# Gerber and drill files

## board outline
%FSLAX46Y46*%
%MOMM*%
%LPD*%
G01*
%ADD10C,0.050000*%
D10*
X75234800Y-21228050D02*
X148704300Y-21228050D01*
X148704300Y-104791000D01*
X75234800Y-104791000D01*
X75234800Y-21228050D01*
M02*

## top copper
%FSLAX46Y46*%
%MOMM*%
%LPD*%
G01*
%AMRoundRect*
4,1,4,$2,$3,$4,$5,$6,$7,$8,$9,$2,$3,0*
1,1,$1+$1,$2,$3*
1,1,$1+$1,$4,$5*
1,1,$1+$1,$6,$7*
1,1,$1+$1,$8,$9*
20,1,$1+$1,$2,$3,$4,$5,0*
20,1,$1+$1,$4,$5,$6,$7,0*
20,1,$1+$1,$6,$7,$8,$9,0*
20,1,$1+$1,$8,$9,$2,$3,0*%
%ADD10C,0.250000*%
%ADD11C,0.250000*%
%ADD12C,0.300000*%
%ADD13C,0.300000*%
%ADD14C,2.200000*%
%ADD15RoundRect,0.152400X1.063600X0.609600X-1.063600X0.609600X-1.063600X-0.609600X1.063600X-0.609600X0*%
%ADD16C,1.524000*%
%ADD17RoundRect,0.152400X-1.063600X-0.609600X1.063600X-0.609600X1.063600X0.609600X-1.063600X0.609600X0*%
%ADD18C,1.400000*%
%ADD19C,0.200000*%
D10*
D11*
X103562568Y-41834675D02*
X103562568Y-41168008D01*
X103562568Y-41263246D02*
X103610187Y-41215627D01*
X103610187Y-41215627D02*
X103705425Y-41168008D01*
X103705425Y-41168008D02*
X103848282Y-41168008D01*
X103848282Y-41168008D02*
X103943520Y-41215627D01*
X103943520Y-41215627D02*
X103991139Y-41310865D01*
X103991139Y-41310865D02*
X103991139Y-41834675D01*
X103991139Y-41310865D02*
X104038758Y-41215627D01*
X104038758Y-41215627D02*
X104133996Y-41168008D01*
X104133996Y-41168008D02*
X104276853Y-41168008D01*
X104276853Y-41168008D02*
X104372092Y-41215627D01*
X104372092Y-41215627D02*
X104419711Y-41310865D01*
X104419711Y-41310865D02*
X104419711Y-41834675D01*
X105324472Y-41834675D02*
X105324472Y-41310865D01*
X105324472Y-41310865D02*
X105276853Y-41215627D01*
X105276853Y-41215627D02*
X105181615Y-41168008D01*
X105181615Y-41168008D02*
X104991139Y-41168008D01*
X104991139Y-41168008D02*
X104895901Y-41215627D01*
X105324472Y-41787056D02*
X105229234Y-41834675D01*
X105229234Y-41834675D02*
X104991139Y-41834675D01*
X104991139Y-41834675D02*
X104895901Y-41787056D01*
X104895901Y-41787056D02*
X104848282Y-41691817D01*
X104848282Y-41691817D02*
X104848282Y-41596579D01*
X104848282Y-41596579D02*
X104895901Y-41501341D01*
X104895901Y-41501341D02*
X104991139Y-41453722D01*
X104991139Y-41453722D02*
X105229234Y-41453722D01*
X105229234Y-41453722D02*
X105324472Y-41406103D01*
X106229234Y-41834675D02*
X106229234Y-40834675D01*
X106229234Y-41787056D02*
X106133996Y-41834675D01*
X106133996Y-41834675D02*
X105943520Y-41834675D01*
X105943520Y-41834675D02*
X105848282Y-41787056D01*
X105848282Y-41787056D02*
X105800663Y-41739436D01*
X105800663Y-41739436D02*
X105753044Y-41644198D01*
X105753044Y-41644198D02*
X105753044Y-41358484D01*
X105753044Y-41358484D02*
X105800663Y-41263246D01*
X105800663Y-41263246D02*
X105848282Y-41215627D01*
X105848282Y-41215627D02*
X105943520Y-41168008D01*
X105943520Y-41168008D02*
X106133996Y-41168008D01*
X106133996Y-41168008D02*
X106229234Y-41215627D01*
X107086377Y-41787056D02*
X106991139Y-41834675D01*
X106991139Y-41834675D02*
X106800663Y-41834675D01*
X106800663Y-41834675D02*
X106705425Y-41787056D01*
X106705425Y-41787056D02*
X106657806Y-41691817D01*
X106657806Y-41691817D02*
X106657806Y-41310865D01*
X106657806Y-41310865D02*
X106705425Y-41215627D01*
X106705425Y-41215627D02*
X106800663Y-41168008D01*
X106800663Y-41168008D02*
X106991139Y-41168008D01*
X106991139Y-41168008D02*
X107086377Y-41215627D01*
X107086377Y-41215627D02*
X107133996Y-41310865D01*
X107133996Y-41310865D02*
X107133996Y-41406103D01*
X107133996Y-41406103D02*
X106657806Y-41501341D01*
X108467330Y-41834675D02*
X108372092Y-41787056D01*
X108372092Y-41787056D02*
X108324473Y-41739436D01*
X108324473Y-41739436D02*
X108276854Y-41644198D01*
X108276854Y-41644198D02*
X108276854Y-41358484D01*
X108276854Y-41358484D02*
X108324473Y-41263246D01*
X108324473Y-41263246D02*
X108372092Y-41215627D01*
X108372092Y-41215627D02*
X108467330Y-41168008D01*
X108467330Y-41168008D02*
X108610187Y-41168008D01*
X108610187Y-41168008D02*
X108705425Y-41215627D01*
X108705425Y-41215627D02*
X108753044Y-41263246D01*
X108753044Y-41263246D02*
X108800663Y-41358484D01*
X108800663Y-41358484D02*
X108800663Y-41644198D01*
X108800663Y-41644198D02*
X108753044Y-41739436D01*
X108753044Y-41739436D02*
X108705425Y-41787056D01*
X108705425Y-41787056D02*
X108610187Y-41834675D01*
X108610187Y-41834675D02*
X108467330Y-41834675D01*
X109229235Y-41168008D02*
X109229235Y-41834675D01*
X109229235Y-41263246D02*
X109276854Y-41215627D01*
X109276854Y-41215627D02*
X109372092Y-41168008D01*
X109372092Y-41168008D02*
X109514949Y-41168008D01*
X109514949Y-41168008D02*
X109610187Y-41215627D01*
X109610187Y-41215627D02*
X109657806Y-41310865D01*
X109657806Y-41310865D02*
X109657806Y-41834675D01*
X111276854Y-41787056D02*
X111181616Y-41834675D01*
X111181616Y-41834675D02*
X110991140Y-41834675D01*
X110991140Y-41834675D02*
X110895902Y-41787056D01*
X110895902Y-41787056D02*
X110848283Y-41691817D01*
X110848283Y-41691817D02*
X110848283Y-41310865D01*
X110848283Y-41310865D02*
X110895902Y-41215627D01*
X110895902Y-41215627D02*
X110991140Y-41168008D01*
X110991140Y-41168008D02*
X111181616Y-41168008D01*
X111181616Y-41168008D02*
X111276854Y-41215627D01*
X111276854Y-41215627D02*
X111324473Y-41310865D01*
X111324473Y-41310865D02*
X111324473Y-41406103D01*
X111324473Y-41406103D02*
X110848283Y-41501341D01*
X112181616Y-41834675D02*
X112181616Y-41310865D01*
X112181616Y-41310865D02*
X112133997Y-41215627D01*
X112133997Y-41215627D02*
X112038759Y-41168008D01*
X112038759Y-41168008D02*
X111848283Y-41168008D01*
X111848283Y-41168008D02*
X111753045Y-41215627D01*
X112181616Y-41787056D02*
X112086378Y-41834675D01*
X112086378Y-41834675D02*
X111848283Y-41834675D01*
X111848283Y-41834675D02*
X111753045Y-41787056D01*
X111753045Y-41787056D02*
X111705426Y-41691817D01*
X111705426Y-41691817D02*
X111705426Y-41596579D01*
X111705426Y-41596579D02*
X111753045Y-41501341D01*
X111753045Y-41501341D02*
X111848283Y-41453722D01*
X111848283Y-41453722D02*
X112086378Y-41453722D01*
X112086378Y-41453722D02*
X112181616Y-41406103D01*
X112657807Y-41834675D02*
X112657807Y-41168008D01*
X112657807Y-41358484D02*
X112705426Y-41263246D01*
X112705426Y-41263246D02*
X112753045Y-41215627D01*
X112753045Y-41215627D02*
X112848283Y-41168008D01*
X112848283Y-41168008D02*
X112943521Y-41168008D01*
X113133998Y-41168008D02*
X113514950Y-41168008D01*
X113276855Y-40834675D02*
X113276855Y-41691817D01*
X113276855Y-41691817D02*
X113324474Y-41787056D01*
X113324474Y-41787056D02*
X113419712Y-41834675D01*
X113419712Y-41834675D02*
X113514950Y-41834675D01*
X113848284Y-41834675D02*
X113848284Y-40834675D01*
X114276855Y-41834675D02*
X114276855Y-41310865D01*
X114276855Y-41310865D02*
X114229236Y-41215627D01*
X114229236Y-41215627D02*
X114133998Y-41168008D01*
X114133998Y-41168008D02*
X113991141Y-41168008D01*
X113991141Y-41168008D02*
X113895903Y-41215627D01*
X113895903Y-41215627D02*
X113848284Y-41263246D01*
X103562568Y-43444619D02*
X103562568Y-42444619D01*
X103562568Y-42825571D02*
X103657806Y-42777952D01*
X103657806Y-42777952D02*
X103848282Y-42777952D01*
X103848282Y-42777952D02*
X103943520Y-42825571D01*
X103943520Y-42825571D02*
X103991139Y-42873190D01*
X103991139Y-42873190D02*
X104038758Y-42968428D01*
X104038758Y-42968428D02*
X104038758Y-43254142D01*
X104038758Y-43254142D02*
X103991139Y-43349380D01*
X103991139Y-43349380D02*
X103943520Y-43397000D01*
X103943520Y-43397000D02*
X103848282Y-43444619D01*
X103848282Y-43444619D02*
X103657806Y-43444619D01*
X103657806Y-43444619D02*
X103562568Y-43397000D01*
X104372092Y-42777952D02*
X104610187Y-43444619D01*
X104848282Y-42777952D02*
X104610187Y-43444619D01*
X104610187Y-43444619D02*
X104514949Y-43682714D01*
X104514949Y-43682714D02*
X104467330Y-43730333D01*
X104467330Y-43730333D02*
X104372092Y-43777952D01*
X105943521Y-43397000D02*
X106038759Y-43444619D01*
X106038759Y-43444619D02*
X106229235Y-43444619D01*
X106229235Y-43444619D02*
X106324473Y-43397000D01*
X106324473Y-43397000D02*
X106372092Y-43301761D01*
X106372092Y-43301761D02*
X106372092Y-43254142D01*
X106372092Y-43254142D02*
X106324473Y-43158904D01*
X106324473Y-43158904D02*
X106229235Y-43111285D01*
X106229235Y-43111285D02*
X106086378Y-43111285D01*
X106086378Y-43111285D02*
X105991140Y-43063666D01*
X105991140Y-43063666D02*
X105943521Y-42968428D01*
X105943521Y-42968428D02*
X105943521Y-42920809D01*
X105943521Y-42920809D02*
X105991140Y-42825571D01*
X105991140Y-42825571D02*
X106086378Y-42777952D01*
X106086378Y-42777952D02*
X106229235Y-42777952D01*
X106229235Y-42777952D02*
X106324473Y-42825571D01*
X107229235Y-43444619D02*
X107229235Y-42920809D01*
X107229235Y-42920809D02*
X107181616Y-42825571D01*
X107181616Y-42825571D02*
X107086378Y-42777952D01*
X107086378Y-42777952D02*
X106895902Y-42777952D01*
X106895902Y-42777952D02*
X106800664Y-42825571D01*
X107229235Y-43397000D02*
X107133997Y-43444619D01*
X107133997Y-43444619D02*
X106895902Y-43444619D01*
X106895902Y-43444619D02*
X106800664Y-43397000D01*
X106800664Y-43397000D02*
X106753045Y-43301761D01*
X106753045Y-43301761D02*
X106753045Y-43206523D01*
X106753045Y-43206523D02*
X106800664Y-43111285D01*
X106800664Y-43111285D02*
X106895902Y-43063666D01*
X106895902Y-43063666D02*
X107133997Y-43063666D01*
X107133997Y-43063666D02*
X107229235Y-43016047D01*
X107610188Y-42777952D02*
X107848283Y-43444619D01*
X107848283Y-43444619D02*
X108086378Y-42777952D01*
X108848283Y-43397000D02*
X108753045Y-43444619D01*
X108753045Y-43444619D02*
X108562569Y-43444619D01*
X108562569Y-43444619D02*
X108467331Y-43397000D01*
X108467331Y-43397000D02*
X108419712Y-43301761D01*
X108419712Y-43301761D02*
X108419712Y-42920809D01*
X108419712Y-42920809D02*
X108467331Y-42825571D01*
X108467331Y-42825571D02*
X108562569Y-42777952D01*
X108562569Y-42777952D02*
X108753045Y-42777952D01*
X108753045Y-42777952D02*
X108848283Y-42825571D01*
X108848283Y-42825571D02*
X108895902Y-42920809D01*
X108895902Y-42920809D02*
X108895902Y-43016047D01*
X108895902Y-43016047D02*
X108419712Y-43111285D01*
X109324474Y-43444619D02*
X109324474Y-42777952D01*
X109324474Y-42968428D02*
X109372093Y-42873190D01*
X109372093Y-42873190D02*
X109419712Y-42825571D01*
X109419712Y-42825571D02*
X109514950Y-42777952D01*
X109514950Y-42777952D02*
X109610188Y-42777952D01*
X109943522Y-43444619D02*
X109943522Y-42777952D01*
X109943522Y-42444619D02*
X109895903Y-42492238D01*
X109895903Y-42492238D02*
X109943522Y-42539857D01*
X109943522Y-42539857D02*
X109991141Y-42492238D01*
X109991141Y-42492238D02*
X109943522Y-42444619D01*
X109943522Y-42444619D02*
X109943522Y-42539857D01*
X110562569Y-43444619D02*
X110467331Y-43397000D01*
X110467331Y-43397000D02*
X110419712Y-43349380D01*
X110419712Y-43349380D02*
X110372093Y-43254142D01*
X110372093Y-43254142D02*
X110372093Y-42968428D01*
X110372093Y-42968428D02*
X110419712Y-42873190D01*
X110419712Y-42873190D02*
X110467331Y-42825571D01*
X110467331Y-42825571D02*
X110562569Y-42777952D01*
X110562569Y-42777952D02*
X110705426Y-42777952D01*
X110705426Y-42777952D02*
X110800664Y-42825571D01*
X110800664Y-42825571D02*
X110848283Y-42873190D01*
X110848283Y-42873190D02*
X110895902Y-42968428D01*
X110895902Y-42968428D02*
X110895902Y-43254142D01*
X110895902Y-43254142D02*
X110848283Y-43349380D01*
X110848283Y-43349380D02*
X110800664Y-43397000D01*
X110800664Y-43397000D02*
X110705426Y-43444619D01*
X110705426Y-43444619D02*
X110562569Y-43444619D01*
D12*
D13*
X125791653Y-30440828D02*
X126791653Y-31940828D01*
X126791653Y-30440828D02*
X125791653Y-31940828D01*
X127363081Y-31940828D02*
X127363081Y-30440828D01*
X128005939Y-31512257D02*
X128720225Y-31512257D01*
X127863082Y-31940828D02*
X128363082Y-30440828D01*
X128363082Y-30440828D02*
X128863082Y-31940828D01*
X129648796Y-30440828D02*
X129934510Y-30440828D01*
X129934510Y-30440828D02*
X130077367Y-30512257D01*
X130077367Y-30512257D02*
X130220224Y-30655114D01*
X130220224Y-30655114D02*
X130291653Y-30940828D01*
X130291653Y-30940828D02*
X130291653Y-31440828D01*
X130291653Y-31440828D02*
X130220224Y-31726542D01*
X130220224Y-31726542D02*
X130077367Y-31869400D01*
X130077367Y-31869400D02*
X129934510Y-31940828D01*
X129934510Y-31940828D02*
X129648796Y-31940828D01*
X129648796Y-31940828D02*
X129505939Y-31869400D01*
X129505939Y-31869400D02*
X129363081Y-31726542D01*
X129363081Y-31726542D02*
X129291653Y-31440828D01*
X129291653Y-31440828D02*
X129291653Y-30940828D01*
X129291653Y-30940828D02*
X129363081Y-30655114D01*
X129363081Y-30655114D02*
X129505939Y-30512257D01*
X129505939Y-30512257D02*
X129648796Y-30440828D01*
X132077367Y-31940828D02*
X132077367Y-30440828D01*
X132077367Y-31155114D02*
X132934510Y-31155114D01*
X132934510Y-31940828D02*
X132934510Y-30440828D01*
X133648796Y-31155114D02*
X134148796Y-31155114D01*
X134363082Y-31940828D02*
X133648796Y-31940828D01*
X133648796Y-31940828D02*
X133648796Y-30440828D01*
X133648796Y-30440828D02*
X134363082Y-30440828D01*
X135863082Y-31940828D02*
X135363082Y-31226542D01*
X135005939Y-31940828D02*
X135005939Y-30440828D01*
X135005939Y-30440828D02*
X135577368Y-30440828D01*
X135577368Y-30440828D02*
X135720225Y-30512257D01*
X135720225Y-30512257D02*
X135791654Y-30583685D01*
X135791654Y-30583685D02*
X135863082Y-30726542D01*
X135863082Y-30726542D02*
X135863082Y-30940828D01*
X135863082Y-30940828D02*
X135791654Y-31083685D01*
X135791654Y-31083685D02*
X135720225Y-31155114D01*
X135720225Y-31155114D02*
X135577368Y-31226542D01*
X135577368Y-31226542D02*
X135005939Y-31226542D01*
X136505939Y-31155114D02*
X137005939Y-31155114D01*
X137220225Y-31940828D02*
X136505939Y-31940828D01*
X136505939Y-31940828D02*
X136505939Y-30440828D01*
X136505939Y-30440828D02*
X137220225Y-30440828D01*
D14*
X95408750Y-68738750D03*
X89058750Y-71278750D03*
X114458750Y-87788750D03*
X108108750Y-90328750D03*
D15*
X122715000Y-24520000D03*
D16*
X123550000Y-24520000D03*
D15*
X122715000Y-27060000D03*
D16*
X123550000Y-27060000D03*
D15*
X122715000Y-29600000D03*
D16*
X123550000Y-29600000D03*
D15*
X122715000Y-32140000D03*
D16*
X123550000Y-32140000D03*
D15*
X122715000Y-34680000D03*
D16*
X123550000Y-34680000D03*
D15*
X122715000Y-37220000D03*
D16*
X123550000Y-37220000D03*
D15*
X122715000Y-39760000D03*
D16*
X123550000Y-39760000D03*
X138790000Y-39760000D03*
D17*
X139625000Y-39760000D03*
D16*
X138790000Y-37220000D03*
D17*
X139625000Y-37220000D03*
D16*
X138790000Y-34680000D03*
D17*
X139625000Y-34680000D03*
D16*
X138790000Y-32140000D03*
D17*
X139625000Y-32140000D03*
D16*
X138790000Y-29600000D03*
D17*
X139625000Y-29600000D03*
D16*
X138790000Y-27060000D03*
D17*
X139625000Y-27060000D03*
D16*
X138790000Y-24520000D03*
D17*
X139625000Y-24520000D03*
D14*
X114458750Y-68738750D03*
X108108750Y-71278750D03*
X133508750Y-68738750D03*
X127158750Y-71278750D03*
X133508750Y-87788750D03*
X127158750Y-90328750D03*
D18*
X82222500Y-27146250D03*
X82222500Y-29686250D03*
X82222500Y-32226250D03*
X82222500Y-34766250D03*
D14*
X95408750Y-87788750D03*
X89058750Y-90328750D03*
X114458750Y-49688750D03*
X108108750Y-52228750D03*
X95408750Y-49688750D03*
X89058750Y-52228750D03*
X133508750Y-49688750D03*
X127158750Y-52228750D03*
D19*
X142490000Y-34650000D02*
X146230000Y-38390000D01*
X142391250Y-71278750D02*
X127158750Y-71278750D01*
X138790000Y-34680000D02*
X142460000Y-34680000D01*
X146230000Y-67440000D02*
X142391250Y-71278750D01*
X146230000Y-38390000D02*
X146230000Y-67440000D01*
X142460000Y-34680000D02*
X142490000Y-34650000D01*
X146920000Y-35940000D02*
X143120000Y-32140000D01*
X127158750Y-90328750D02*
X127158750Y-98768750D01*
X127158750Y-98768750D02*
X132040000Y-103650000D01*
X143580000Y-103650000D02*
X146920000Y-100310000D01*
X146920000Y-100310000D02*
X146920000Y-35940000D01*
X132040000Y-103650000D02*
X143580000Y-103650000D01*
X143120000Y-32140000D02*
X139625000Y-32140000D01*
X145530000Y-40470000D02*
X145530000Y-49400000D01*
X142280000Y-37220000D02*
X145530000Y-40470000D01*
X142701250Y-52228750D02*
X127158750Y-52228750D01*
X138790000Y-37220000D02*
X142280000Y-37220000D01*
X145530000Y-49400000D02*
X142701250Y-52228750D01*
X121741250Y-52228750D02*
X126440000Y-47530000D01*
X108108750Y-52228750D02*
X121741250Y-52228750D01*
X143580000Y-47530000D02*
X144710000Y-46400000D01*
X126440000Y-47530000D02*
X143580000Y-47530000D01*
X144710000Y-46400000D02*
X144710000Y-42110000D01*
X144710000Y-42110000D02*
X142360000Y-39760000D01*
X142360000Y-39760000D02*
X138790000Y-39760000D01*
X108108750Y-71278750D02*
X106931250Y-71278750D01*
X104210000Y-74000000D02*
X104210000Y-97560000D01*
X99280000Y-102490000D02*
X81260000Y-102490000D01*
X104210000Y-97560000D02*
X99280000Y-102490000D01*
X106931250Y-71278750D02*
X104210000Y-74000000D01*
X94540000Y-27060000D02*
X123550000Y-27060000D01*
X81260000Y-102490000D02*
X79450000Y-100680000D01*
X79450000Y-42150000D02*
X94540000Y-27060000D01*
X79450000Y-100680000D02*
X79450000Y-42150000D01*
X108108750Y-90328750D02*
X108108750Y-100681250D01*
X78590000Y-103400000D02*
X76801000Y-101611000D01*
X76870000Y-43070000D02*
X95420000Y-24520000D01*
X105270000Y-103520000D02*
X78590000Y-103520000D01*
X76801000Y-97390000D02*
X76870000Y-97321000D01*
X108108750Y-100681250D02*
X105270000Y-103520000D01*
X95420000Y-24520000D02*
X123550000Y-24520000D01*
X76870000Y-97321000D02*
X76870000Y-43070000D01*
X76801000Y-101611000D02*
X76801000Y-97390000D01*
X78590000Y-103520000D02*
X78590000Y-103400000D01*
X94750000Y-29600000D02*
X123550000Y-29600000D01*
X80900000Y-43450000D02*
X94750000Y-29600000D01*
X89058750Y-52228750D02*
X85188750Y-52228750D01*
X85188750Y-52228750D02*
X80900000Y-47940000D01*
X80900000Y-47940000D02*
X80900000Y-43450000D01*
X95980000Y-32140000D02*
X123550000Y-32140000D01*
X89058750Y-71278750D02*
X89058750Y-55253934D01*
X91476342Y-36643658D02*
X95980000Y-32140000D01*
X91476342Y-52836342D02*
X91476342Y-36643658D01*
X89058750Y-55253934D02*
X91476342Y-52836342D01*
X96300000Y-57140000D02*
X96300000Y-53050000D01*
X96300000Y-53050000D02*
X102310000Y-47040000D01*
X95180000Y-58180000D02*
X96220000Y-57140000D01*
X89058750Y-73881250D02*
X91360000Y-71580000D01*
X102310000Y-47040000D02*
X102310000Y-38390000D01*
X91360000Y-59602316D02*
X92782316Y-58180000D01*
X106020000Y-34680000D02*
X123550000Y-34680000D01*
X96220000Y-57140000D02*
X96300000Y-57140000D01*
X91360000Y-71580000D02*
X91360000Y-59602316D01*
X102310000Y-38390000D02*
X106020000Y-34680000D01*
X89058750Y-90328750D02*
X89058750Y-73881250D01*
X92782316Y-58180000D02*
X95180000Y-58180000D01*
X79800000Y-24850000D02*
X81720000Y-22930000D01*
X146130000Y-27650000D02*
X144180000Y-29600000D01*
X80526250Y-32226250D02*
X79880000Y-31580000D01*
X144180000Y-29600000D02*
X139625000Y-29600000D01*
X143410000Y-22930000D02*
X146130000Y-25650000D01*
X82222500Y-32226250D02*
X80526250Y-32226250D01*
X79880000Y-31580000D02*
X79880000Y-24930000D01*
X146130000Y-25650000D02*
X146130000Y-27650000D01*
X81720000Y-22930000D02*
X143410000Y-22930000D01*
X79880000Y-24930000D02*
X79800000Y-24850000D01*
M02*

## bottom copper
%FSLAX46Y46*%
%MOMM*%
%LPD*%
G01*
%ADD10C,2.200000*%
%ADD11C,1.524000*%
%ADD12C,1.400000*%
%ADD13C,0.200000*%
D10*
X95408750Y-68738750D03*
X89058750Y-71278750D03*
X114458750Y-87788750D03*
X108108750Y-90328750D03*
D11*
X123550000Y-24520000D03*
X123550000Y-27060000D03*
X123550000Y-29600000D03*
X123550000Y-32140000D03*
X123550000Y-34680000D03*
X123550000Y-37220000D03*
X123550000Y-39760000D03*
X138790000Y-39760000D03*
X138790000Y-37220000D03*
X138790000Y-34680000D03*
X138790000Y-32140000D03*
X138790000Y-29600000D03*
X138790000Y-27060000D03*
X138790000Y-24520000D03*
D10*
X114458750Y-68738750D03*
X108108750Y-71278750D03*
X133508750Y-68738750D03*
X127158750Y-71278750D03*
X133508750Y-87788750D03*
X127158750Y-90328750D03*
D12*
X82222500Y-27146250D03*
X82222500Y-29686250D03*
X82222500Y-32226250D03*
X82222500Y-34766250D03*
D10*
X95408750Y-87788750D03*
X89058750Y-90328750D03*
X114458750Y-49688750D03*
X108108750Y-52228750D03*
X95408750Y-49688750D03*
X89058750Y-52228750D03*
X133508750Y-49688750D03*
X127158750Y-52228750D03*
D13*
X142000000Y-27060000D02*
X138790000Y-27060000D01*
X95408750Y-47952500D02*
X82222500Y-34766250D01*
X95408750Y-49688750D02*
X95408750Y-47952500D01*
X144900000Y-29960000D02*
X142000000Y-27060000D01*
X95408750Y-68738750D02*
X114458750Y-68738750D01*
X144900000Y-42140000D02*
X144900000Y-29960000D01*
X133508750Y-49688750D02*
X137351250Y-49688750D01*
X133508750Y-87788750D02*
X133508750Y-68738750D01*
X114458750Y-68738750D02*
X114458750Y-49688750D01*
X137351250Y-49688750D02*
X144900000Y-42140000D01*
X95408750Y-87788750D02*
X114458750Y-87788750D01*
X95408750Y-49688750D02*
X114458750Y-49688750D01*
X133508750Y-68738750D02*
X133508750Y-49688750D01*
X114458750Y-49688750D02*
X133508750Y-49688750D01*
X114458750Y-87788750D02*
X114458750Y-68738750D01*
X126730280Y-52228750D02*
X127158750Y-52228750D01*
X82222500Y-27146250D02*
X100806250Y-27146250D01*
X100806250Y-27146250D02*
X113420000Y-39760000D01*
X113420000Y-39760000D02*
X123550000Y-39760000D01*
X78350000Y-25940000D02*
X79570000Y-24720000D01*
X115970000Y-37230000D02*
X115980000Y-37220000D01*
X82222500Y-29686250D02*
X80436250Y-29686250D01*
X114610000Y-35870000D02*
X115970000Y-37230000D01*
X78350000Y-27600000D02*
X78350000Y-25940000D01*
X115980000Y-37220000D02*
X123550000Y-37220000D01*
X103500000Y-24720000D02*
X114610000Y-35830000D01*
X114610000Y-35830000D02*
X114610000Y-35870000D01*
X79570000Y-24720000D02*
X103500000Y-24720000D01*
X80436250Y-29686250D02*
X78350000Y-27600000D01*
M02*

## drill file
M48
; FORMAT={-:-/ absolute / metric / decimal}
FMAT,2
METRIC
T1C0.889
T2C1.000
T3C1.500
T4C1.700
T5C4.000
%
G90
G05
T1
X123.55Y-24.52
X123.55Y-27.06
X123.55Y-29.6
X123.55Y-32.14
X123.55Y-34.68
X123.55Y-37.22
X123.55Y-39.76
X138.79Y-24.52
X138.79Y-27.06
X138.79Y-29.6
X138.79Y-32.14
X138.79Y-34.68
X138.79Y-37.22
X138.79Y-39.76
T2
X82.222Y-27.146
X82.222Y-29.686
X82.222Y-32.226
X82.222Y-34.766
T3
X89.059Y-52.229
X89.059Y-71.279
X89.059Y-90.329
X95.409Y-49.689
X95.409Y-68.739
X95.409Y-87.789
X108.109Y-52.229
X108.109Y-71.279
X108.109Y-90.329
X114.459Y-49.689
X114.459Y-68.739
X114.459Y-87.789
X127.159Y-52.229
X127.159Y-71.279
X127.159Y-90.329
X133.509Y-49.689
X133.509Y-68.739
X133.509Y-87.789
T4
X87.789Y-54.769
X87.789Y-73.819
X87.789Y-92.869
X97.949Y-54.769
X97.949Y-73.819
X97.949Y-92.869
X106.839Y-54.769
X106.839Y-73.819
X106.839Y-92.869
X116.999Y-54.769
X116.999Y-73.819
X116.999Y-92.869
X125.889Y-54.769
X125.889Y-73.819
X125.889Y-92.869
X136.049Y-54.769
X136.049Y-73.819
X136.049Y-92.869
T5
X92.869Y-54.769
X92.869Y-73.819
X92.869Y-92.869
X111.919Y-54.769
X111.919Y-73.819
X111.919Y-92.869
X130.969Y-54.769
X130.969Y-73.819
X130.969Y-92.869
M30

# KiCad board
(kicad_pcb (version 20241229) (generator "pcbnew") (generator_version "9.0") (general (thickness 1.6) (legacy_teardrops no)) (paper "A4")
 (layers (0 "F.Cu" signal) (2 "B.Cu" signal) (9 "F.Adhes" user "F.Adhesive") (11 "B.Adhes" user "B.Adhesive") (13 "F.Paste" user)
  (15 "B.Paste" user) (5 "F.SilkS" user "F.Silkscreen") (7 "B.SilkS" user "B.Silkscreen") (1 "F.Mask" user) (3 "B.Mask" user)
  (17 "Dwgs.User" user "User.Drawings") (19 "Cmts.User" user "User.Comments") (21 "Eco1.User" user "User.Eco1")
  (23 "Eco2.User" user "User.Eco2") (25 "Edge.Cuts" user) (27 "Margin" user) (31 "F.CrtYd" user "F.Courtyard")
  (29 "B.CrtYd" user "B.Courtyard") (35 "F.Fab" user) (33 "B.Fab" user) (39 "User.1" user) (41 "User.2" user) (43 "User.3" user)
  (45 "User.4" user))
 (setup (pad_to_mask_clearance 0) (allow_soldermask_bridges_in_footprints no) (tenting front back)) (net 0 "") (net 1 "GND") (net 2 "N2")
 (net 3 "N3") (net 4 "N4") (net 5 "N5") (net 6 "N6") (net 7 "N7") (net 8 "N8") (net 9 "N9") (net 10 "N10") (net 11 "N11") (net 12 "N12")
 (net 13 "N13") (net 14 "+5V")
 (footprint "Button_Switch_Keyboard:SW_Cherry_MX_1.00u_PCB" (layer "F.Cu") (at 95.40875 68.73875)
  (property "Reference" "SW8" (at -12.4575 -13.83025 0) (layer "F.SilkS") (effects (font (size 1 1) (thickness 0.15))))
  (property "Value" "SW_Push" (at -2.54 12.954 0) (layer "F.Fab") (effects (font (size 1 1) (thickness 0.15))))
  (pad "" np_thru_hole circle (at -7.62 5.08) (size 1.7 1.7) (drill 1.7) (layers "*.Cu" "*.Mask"))
  (pad "" np_thru_hole circle (at -2.54 5.08) (size 4 4) (drill 4) (layers "*.Cu" "*.Mask"))
  (pad "" np_thru_hole circle (at 2.54 5.08) (size 1.7 1.7) (drill 1.7) (layers "*.Cu" "*.Mask"))
  (pad "1" thru_hole circle (at 0 0) (size 2.2 2.2) (drill 1.5) (layers "*.Cu" "*.Mask") (remove_unused_layers no) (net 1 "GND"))
  (pad "2" thru_hole circle (at -6.35 2.54) (size 2.2 2.2) (drill 1.5) (layers "*.Cu" "*.Mask") (remove_unused_layers no) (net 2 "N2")))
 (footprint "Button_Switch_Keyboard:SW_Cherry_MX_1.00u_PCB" (layer "F.Cu") (at 114.45875 87.78875)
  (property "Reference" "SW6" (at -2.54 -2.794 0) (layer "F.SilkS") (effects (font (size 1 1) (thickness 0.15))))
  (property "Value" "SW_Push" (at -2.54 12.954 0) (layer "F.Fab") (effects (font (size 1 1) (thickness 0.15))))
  (pad "" np_thru_hole circle (at -7.62 5.08) (size 1.7 1.7) (drill 1.7) (layers "*.Cu" "*.Mask"))
  (pad "" np_thru_hole circle (at -2.54 5.08) (size 4 4) (drill 4) (layers "*.Cu" "*.Mask"))
  (pad "" np_thru_hole circle (at 2.54 5.08) (size 1.7 1.7) (drill 1.7) (layers "*.Cu" "*.Mask"))
  (pad "1" thru_hole circle (at 0 0) (size 2.2 2.2) (drill 1.5) (layers "*.Cu" "*.Mask") (remove_unused_layers no) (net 1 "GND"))
  (pad "2" thru_hole circle (at -6.35 2.54) (size 2.2 2.2) (drill 1.5) (layers "*.Cu" "*.Mask") (remove_unused_layers no) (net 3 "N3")))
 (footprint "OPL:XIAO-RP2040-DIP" (layer "F.Cu") (at 131.17 32.14)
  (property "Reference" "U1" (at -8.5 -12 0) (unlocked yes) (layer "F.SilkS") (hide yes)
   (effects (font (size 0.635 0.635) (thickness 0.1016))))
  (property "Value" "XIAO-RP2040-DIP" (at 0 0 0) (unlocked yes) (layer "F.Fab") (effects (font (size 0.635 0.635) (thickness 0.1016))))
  (pad "1" smd roundrect (at -8.455 -7.62 180) (size 2.432 1.524) (layers "F.Cu" "F.Mask") (roundrect_rratio 0.1) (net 3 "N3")
   (thermal_bridge_angle 45))
  (pad "1" thru_hole circle (at -7.62 -7.62 180) (size 1.524 1.524) (drill 0.889) (layers "*.Cu" "*.Mask") (remove_unused_layers no)
   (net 3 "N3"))
  (pad "2" smd roundrect (at -8.455 -5.08 180) (size 2.432 1.524) (layers "F.Cu" "F.Mask") (roundrect_rratio 0.1) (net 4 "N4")
   (thermal_bridge_angle 45))
  (pad "2" thru_hole circle (at -7.62 -5.08 180) (size 1.524 1.524) (drill 0.889) (layers "*.Cu" "*.Mask") (remove_unused_layers no)
   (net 4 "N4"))
  (pad "3" smd roundrect (at -8.455 -2.54 180) (size 2.432 1.524) (layers "F.Cu" "F.Mask") (roundrect_rratio 0.1) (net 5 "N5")
   (thermal_bridge_angle 45))
  (pad "3" thru_hole circle (at -7.62 -2.54 180) (size 1.524 1.524) (drill 0.889) (layers "*.Cu" "*.Mask") (remove_unused_layers no)
   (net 5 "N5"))
  (pad "4" smd roundrect (at -8.455 0 180) (size 2.432 1.524) (layers "F.Cu" "F.Mask") (roundrect_rratio 0.1) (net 2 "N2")
   (thermal_bridge_angle 45))
  (pad "4" thru_hole circle (at -7.62 0 180) (size 1.524 1.524) (drill 0.889) (layers "*.Cu" "*.Mask") (remove_unused_layers no)
   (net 2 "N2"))
  (pad "5" smd roundrect (at -8.455 2.54 180) (size 2.432 1.524) (layers "F.Cu" "F.Mask") (roundrect_rratio 0.1) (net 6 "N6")
   (thermal_bridge_angle 45))
  (pad "5" thru_hole circle (at -7.62 2.54 180) (size 1.524 1.524) (drill 0.889) (layers "*.Cu" "*.Mask") (remove_unused_layers no)
   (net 6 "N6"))
  (pad "6" smd roundrect (at -8.455 5.08 180) (size 2.432 1.524) (layers "F.Cu" "F.Mask") (roundrect_rratio 0.1) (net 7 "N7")
   (thermal_bridge_angle 45))
  (pad "6" thru_hole circle (at -7.62 5.08 180) (size 1.524 1.524) (drill 0.889) (layers "*.Cu" "*.Mask") (remove_unused_layers no)
   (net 7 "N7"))
  (pad "7" smd roundrect (at -8.455 7.62 180) (size 2.432 1.524) (layers "F.Cu" "F.Mask") (roundrect_rratio 0.1) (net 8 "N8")
   (thermal_bridge_angle 45))
  (pad "7" thru_hole circle (at -7.62 7.62 180) (size 1.524 1.524) (drill 0.889) (layers "*.Cu" "*.Mask") (remove_unused_layers no)
   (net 8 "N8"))
  (pad "8" thru_hole circle (at 7.62 7.62) (size 1.524 1.524) (drill 0.889) (layers "*.Cu" "*.Mask") (remove_unused_layers no) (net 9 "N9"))
  (pad "8" smd roundrect (at 8.455 7.62) (size 2.432 1.524) (layers "F.Cu" "F.Mask") (roundrect_rratio 0.1) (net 9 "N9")
   (thermal_bridge_angle 45))
  (pad "9" thru_hole circle (at 7.62 5.08) (size 1.524 1.524) (drill 0.889) (layers "*.Cu" "*.Mask") (remove_unused_layers no)
   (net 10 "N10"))
  (pad "9" smd roundrect (at 8.455 5.08) (size 2.432 1.524) (layers "F.Cu" "F.Mask") (roundrect_rratio 0.1) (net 10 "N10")
   (thermal_bridge_angle 45))
  (pad "10" thru_hole circle (at 7.62 2.54) (size 1.524 1.524) (drill 0.889) (layers "*.Cu" "*.Mask") (remove_unused_layers no)
   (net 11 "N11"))
  (pad "10" smd roundrect (at 8.455 2.54) (size 2.432 1.524) (layers "F.Cu" "F.Mask") (roundrect_rratio 0.1) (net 11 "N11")
   (thermal_bridge_angle 45))
  (pad "11" thru_hole circle (at 7.62 0) (size 1.524 1.524) (drill 0.889) (layers "*.Cu" "*.Mask") (remove_unused_layers no) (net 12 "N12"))
  (pad "11" smd roundrect (at 8.455 0) (size 2.432 1.524) (layers "F.Cu" "F.Mask") (roundrect_rratio 0.1) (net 12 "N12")
   (thermal_bridge_angle 45))
  (pad "12" thru_hole circle (at 7.62 -2.54) (size 1.524 1.524) (drill 0.889) (layers "*.Cu" "*.Mask") (remove_unused_layers no)
   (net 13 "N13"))
  (pad "12" smd roundrect (at 8.455 -2.54) (size 2.432 1.524) (layers "F.Cu" "F.Mask") (roundrect_rratio 0.1) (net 13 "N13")
   (thermal_bridge_angle 45))
  (pad "13" thru_hole circle (at 7.62 -5.08) (size 1.524 1.524) (drill 0.889) (layers "*.Cu" "*.Mask") (remove_unused_layers no)
   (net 1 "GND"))
  (pad "13" smd roundrect (at 8.455 -5.08) (size 2.432 1.524) (layers "F.Cu" "F.Mask") (roundrect_rratio 0.1) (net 1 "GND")
   (thermal_bridge_angle 45))
  (pad "14" thru_hole circle (at 7.62 -7.62) (size 1.524 1.524) (drill 0.889) (layers "*.Cu" "*.Mask") (remove_unused_layers no)
   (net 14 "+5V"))
  (pad "14" smd roundrect (at 8.455 -7.62) (size 2.432 1.524) (layers "F.Cu" "F.Mask") (roundrect_rratio 0.1) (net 14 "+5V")
   (thermal_bridge_angle 45)))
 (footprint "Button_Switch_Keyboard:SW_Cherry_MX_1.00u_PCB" (layer "F.Cu") (at 114.45875 68.73875)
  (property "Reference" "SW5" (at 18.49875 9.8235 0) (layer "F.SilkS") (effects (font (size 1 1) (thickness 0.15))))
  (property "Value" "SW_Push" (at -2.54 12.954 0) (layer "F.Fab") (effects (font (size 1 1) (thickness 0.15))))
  (pad "" np_thru_hole circle (at -7.62 5.08) (size 1.7 1.7) (drill 1.7) (layers "*.Cu" "*.Mask"))
  (pad "" np_thru_hole circle (at -2.54 5.08) (size 4 4) (drill 4) (layers "*.Cu" "*.Mask"))
  (pad "" np_thru_hole circle (at 2.54 5.08) (size 1.7 1.7) (drill 1.7) (layers "*.Cu" "*.Mask"))
  (pad "1" thru_hole circle (at 0 0) (size 2.2 2.2) (drill 1.5) (layers "*.Cu" "*.Mask") (remove_unused_layers no) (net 1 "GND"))
  (pad "2" thru_hole circle (at -6.35 2.54) (size 2.2 2.2) (drill 1.5) (layers "*.Cu" "*.Mask") (remove_unused_layers no) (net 4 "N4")))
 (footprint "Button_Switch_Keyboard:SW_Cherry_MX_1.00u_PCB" (layer "F.Cu") (at 133.50875 68.73875)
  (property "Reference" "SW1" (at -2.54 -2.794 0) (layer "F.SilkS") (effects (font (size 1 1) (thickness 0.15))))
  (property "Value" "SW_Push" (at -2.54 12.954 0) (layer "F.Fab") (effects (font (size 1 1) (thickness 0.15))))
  (pad "" np_thru_hole circle (at -7.62 5.08) (size 1.7 1.7) (drill 1.7) (layers "*.Cu" "*.Mask"))
  (pad "" np_thru_hole circle (at -2.54 5.08) (size 4 4) (drill 4) (layers "*.Cu" "*.Mask"))
  (pad "" np_thru_hole circle (at 2.54 5.08) (size 1.7 1.7) (drill 1.7) (layers "*.Cu" "*.Mask"))
  (pad "1" thru_hole circle (at 0 0) (size 2.2 2.2) (drill 1.5) (layers "*.Cu" "*.Mask") (remove_unused_layers no) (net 1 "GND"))
  (pad "2" thru_hole circle (at -6.35 2.54) (size 2.2 2.2) (drill 1.5) (layers "*.Cu" "*.Mask") (remove_unused_layers no) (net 11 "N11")))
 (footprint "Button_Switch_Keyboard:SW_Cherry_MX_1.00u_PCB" (layer "F.Cu") (at 133.50875 87.78875)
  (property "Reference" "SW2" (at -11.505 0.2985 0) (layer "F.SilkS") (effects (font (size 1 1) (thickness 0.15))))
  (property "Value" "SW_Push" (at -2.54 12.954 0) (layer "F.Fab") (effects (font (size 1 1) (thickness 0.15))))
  (pad "" np_thru_hole circle (at -7.62 5.08) (size 1.7 1.7) (drill 1.7) (layers "*.Cu" "*.Mask"))
  (pad "" np_thru_hole circle (at -2.54 5.08) (size 4 4) (drill 4) (layers "*.Cu" "*.Mask"))
  (pad "" np_thru_hole circle (at 2.54 5.08) (size 1.7 1.7) (drill 1.7) (layers "*.Cu" "*.Mask"))
  (pad "1" thru_hole circle (at 0 0) (size 2.2 2.2) (drill 1.5) (layers "*.Cu" "*.Mask") (remove_unused_layers no) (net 1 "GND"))
  (pad "2" thru_hole circle (at -6.35 2.54) (size 2.2 2.2) (drill 1.5) (layers "*.Cu" "*.Mask") (remove_unused_layers no) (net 12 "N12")))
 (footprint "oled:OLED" (layer "F.Cu") (at 82.2225 30.95625 -90)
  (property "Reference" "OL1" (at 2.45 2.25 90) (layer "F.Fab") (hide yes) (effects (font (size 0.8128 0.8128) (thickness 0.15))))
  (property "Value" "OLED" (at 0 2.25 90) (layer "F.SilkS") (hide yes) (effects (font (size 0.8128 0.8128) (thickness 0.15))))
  (pad "1" thru_hole circle (at -3.81 0 270) (size 1.4 1.4) (drill 1) (layers "*.Cu" "*.Mask") (remove_unused_layers no) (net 8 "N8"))
  (pad "2" thru_hole circle (at -1.27 0 270) (size 1.4 1.4) (drill 1) (layers "*.Cu" "*.Mask") (remove_unused_layers no) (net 7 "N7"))
  (pad "3" thru_hole circle (at 1.27 0 270) (size 1.4 1.4) (drill 1) (layers "*.Cu" "*.Mask") (remove_unused_layers no) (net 13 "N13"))
  (pad "4" thru_hole circle (at 3.81 0 270) (size 1.4 1.4) (drill 1) (layers "*.Cu" "*.Mask") (remove_unused_layers no) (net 1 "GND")))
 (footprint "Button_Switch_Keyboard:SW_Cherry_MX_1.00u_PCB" (layer "F.Cu") (at 95.40875 87.78875)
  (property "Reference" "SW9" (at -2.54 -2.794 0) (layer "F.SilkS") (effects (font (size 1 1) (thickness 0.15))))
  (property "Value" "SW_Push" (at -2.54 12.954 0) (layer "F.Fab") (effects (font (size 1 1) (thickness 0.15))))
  (pad "" np_thru_hole circle (at -7.62 5.08) (size 1.7 1.7) (drill 1.7) (layers "*.Cu" "*.Mask"))
  (pad "" np_thru_hole circle (at -2.54 5.08) (size 4 4) (drill 4) (layers "*.Cu" "*.Mask"))
  (pad "" np_thru_hole circle (at 2.54 5.08) (size 1.7 1.7) (drill 1.7) (layers "*.Cu" "*.Mask"))
  (pad "1" thru_hole circle (at 0 0) (size 2.2 2.2) (drill 1.5) (layers "*.Cu" "*.Mask") (remove_unused_layers no) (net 1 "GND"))
  (pad "2" thru_hole circle (at -6.35 2.54) (size 2.2 2.2) (drill 1.5) (layers "*.Cu" "*.Mask") (remove_unused_layers no) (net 6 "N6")))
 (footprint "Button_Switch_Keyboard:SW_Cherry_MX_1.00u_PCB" (layer "F.Cu") (at 114.45875 49.68875)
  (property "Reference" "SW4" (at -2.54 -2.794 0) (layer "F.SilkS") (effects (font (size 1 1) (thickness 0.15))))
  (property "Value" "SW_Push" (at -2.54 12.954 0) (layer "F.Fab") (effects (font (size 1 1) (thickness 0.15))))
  (pad "" np_thru_hole circle (at -7.62 5.08) (size 1.7 1.7) (drill 1.7) (layers "*.Cu" "*.Mask"))
  (pad "" np_thru_hole circle (at -2.54 5.08) (size 4 4) (drill 4) (layers "*.Cu" "*.Mask"))
  (pad "" np_thru_hole circle (at 2.54 5.08) (size 1.7 1.7) (drill 1.7) (layers "*.Cu" "*.Mask"))
  (pad "1" thru_hole circle (at 0 0) (size 2.2 2.2) (drill 1.5) (layers "*.Cu" "*.Mask") (remove_unused_layers no) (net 1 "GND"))
  (pad "2" thru_hole circle (at -6.35 2.54) (size 2.2 2.2) (drill 1.5) (layers "*.Cu" "*.Mask") (remove_unused_layers no) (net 9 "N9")))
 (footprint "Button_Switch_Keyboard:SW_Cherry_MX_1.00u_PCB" (layer "F.Cu") (at 95.40875 49.68875)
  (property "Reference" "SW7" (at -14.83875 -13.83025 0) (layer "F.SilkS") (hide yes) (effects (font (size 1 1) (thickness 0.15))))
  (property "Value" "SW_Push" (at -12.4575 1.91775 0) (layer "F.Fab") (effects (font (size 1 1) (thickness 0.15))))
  (pad "" np_thru_hole circle (at -7.62 5.08) (size 1.7 1.7) (drill 1.7) (layers "*.Cu" "*.Mask"))
  (pad "" np_thru_hole circle (at -2.54 5.08) (size 4 4) (drill 4) (layers "*.Cu" "*.Mask"))
  (pad "" np_thru_hole circle (at 2.54 5.08) (size 1.7 1.7) (drill 1.7) (layers "*.Cu" "*.Mask"))
  (pad "1" thru_hole circle (at 0 0) (size 2.2 2.2) (drill 1.5) (layers "*.Cu" "*.Mask") (remove_unused_layers no) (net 1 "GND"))
  (pad "2" thru_hole circle (at -6.35 2.54) (size 2.2 2.2) (drill 1.5) (layers "*.Cu" "*.Mask") (remove_unused_layers no) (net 5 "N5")))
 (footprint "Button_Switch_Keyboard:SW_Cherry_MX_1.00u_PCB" (layer "F.Cu") (at 133.50875 49.68875)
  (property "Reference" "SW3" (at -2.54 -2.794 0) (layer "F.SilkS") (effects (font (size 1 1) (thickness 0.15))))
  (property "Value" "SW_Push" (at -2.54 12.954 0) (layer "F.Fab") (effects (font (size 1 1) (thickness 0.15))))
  (pad "" np_thru_hole circle (at -7.62 5.08) (size 1.7 1.7) (drill 1.7) (layers "*.Cu" "*.Mask"))
  (pad "" np_thru_hole circle (at -2.54 5.08) (size 4 4) (drill 4) (layers "*.Cu" "*.Mask"))
  (pad "" np_thru_hole circle (at 2.54 5.08) (size 1.7 1.7) (drill 1.7) (layers "*.Cu" "*.Mask"))
  (pad "1" thru_hole circle (at 0 0) (size 2.2 2.2) (drill 1.5) (layers "*.Cu" "*.Mask") (remove_unused_layers no) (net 1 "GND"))
  (pad "2" thru_hole circle (at -6.35 2.54) (size 2.2 2.2) (drill 1.5) (layers "*.Cu" "*.Mask") (remove_unused_layers no) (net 10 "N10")))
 (gr_rect (start 75.2348 21.22805) (end 148.7043 104.791) (stroke (width 0.05) (type default)) (fill no) (layer "Edge.Cuts"))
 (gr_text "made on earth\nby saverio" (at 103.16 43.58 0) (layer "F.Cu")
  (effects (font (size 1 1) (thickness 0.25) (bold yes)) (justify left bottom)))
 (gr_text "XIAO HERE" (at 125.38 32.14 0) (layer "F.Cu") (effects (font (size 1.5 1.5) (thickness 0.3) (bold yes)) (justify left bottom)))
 (segment (start 142 27.06) (end 138.79 27.06) (width 0.2) (layer "B.Cu") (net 1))
 (segment (start 95.40875 47.9525) (end 82.2225 34.76625) (width 0.2) (layer "B.Cu") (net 1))
 (segment (start 95.40875 49.68875) (end 95.40875 47.9525) (width 0.2) (layer "B.Cu") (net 1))
 (segment (start 144.9 29.96) (end 142 27.06) (width 0.2) (layer "B.Cu") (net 1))
 (segment (start 95.40875 68.73875) (end 114.45875 68.73875) (width 0.2) (layer "B.Cu") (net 1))
 (segment (start 144.9 42.14) (end 144.9 29.96) (width 0.2) (layer "B.Cu") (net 1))
 (segment (start 133.50875 49.68875) (end 137.35125 49.68875) (width 0.2) (layer "B.Cu") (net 1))
 (segment (start 133.50875 87.78875) (end 133.50875 68.73875) (width 0.2) (layer "B.Cu") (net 1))
 (segment (start 114.45875 68.73875) (end 114.45875 49.68875) (width 0.2) (layer "B.Cu") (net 1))
 (segment (start 137.35125 49.68875) (end 144.9 42.14) (width 0.2) (layer "B.Cu") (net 1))
 (segment (start 95.40875 87.78875) (end 114.45875 87.78875) (width 0.2) (layer "B.Cu") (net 1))
 (segment (start 95.40875 49.68875) (end 114.45875 49.68875) (width 0.2) (layer "B.Cu") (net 1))
 (segment (start 133.50875 68.73875) (end 133.50875 49.68875) (width 0.2) (layer "B.Cu") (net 1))
 (segment (start 114.45875 49.68875) (end 133.50875 49.68875) (width 0.2) (layer "B.Cu") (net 1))
 (segment (start 114.45875 87.78875) (end 114.45875 68.73875) (width 0.2) (layer "B.Cu") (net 1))
 (segment (start 142.49 34.65) (end 146.23 38.39) (width 0.2) (layer "F.Cu") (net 11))
 (segment (start 142.39125 71.27875) (end 127.15875 71.27875) (width 0.2) (layer "F.Cu") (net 11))
 (segment (start 138.79 34.68) (end 142.46 34.68) (width 0.2) (layer "F.Cu") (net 11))
 (segment (start 146.23 67.44) (end 142.39125 71.27875) (width 0.2) (layer "F.Cu") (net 11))
 (segment (start 146.23 38.39) (end 146.23 67.44) (width 0.2) (layer "F.Cu") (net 11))
 (segment (start 142.46 34.68) (end 142.49 34.65) (width 0.2) (layer "F.Cu") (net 11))
 (segment (start 146.92 35.94) (end 143.12 32.14) (width 0.2) (layer "F.Cu") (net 12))
 (segment (start 127.15875 90.32875) (end 127.15875 98.76875) (width 0.2) (layer "F.Cu") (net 12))
 (segment (start 127.15875 98.76875) (end 132.04 103.65) (width 0.2) (layer "F.Cu") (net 12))
 (segment (start 143.58 103.65) (end 146.92 100.31) (width 0.2) (layer "F.Cu") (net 12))
 (segment (start 146.92 100.31) (end 146.92 35.94) (width 0.2) (layer "F.Cu") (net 12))
 (segment (start 132.04 103.65) (end 143.58 103.65) (width 0.2) (layer "F.Cu") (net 12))
 (segment (start 143.12 32.14) (end 139.625 32.14) (width 0.2) (layer "F.Cu") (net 12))
 (segment (start 145.53 40.47) (end 145.53 49.4) (width 0.2) (layer "F.Cu") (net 10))
 (segment (start 142.28 37.22) (end 145.53 40.47) (width 0.2) (layer "F.Cu") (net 10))
 (segment (start 142.70125 52.22875) (end 127.15875 52.22875) (width 0.2) (layer "F.Cu") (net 10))
 (segment (start 138.79 37.22) (end 142.28 37.22) (width 0.2) (layer "F.Cu") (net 10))
 (segment (start 145.53 49.4) (end 142.70125 52.22875) (width 0.2) (layer "F.Cu") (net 10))
 (segment (start 126.73028 52.22875) (end 127.15875 52.22875) (width 0.2) (layer "B.Cu") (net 10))
 (segment (start 121.74125 52.22875) (end 126.44 47.53) (width 0.2) (layer "F.Cu") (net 9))
 (segment (start 108.10875 52.22875) (end 121.74125 52.22875) (width 0.2) (layer "F.Cu") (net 9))
 (segment (start 143.58 47.53) (end 144.71 46.4) (width 0.2) (layer "F.Cu") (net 9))
 (segment (start 126.44 47.53) (end 143.58 47.53) (width 0.2) (layer "F.Cu") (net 9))
 (segment (start 144.71 46.4) (end 144.71 42.11) (width 0.2) (layer "F.Cu") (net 9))
 (segment (start 144.71 42.11) (end 142.36 39.76) (width 0.2) (layer "F.Cu") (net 9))
 (segment (start 142.36 39.76) (end 138.79 39.76) (width 0.2) (layer "F.Cu") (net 9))
 (segment (start 108.10875 71.27875) (end 106.93125 71.27875) (width 0.2) (layer "F.Cu") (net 4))
 (segment (start 104.21 74) (end 104.21 97.56) (width 0.2) (layer "F.Cu") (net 4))
 (segment (start 99.28 102.49) (end 81.26 102.49) (width 0.2) (layer "F.Cu") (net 4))
 (segment (start 104.21 97.56) (end 99.28 102.49) (width 0.2) (layer "F.Cu") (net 4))
 (segment (start 106.93125 71.27875) (end 104.21 74) (width 0.2) (layer "F.Cu") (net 4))
 (segment (start 94.54 27.06) (end 123.55 27.06) (width 0.2) (layer "F.Cu") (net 4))
 (segment (start 81.26 102.49) (end 79.45 100.68) (width 0.2) (layer "F.Cu") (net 4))
 (segment (start 79.45 42.15) (end 94.54 27.06) (width 0.2) (layer "F.Cu") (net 4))
 (segment (start 79.45 100.68) (end 79.45 42.15) (width 0.2) (layer "F.Cu") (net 4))
 (segment (start 108.10875 90.32875) (end 108.10875 100.68125) (width 0.2) (layer "F.Cu") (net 3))
 (segment (start 78.59 103.4) (end 76.801 101.611) (width 0.2) (layer "F.Cu") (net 3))
 (segment (start 76.87 43.07) (end 95.42 24.52) (width 0.2) (layer "F.Cu") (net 3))
 (segment (start 105.27 103.52) (end 78.59 103.52) (width 0.2) (layer "F.Cu") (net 3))
 (segment (start 76.801 97.39) (end 76.87 97.321) (width 0.2) (layer "F.Cu") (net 3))
 (segment (start 108.10875 100.68125) (end 105.27 103.52) (width 0.2) (layer "F.Cu") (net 3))
 (segment (start 95.42 24.52) (end 123.55 24.52) (width 0.2) (layer "F.Cu") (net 3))
 (segment (start 76.87 97.321) (end 76.87 43.07) (width 0.2) (layer "F.Cu") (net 3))
 (segment (start 76.801 101.611) (end 76.801 97.39) (width 0.2) (layer "F.Cu") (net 3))
 (segment (start 78.59 103.52) (end 78.59 103.4) (width 0.2) (layer "F.Cu") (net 3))
 (segment (start 94.75 29.6) (end 123.55 29.6) (width 0.2) (layer "F.Cu") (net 5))
 (segment (start 80.9 43.45) (end 94.75 29.6) (width 0.2) (layer "F.Cu") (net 5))
 (segment (start 89.05875 52.22875) (end 85.18875 52.22875) (width 0.2) (layer "F.Cu") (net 5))
 (segment (start 85.18875 52.22875) (end 80.9 47.94) (width 0.2) (layer "F.Cu") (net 5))
 (segment (start 80.9 47.94) (end 80.9 43.45) (width 0.2) (layer "F.Cu") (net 5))
 (segment (start 95.98 32.14) (end 123.55 32.14) (width 0.2) (layer "F.Cu") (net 2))
 (segment (start 89.05875 71.27875) (end 89.05875 55.253934) (width 0.2) (layer "F.Cu") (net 2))
 (segment (start 91.476342 36.643658) (end 95.98 32.14) (width 0.2) (layer "F.Cu") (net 2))
 (segment (start 91.476342 52.836342) (end 91.476342 36.643658) (width 0.2) (layer "F.Cu") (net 2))
 (segment (start 89.05875 55.253934) (end 91.476342 52.836342) (width 0.2) (layer "F.Cu") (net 2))
 (segment (start 96.3 57.14) (end 96.3 53.05) (width 0.2) (layer "F.Cu") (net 6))
 (segment (start 96.3 53.05) (end 102.31 47.04) (width 0.2) (layer "F.Cu") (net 6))
 (segment (start 95.18 58.18) (end 96.22 57.14) (width 0.2) (layer "F.Cu") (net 6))
 (segment (start 89.05875 73.88125) (end 91.36 71.58) (width 0.2) (layer "F.Cu") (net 6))
 (segment (start 102.31 47.04) (end 102.31 38.39) (width 0.2) (layer "F.Cu") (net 6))
 (segment (start 91.36 59.602316) (end 92.782316 58.18) (width 0.2) (layer "F.Cu") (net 6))
 (segment (start 106.02 34.68) (end 123.55 34.68) (width 0.2) (layer "F.Cu") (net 6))
 (segment (start 96.22 57.14) (end 96.3 57.14) (width 0.2) (layer "F.Cu") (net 6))
 (segment (start 91.36 71.58) (end 91.36 59.602316) (width 0.2) (layer "F.Cu") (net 6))
 (segment (start 102.31 38.39) (end 106.02 34.68) (width 0.2) (layer "F.Cu") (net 6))
 (segment (start 89.05875 90.32875) (end 89.05875 73.88125) (width 0.2) (layer "F.Cu") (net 6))
 (segment (start 92.782316 58.18) (end 95.18 58.18) (width 0.2) (layer "F.Cu") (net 6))
 (segment (start 82.2225 27.14625) (end 100.80625 27.14625) (width 0.2) (layer "B.Cu") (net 8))
 (segment (start 100.80625 27.14625) (end 113.42 39.76) (width 0.2) (layer "B.Cu") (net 8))
 (segment (start 113.42 39.76) (end 123.55 39.76) (width 0.2) (layer "B.Cu") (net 8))
 (segment (start 79.8 24.85) (end 81.72 22.93) (width 0.2) (layer "F.Cu") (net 13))
 (segment (start 146.13 27.65) (end 144.18 29.6) (width 0.2) (layer "F.Cu") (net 13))
 (segment (start 80.52625 32.22625) (end 79.88 31.58) (width 0.2) (layer "F.Cu") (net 13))
 (segment (start 144.18 29.6) (end 139.625 29.6) (width 0.2) (layer "F.Cu") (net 13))
 (segment (start 143.41 22.93) (end 146.13 25.65) (width 0.2) (layer "F.Cu") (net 13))
 (segment (start 82.2225 32.22625) (end 80.52625 32.22625) (width 0.2) (layer "F.Cu") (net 13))
 (segment (start 79.88 31.58) (end 79.88 24.93) (width 0.2) (layer "F.Cu") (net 13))
 (segment (start 146.13 25.65) (end 146.13 27.65) (width 0.2) (layer "F.Cu") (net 13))
 (segment (start 81.72 22.93) (end 143.41 22.93) (width 0.2) (layer "F.Cu") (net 13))
 (segment (start 79.88 24.93) (end 79.8 24.85) (width 0.2) (layer "F.Cu") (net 13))
 (segment (start 78.35 25.94) (end 79.57 24.72) (width 0.2) (layer "B.Cu") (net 7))
 (segment (start 115.97 37.23) (end 115.98 37.22) (width 0.2) (layer "B.Cu") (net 7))
 (segment (start 82.2225 29.68625) (end 80.43625 29.68625) (width 0.2) (layer "B.Cu") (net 7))
 (segment (start 114.61 35.87) (end 115.97 37.23) (width 0.2) (layer "B.Cu") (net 7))
 (segment (start 78.35 27.6) (end 78.35 25.94) (width 0.2) (layer "B.Cu") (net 7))
 (segment (start 115.98 37.22) (end 123.55 37.22) (width 0.2) (layer "B.Cu") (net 7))
 (segment (start 103.5 24.72) (end 114.61 35.83) (width 0.2) (layer "B.Cu") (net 7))
 (segment (start 114.61 35.83) (end 114.61 35.87) (width 0.2) (layer "B.Cu") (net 7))
 (segment (start 79.57 24.72) (end 103.5 24.72) (width 0.2) (layer "B.Cu") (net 7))
 (segment (start 80.43625 29.68625) (end 78.35 27.6) (width 0.2) (layer "B.Cu") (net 7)))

